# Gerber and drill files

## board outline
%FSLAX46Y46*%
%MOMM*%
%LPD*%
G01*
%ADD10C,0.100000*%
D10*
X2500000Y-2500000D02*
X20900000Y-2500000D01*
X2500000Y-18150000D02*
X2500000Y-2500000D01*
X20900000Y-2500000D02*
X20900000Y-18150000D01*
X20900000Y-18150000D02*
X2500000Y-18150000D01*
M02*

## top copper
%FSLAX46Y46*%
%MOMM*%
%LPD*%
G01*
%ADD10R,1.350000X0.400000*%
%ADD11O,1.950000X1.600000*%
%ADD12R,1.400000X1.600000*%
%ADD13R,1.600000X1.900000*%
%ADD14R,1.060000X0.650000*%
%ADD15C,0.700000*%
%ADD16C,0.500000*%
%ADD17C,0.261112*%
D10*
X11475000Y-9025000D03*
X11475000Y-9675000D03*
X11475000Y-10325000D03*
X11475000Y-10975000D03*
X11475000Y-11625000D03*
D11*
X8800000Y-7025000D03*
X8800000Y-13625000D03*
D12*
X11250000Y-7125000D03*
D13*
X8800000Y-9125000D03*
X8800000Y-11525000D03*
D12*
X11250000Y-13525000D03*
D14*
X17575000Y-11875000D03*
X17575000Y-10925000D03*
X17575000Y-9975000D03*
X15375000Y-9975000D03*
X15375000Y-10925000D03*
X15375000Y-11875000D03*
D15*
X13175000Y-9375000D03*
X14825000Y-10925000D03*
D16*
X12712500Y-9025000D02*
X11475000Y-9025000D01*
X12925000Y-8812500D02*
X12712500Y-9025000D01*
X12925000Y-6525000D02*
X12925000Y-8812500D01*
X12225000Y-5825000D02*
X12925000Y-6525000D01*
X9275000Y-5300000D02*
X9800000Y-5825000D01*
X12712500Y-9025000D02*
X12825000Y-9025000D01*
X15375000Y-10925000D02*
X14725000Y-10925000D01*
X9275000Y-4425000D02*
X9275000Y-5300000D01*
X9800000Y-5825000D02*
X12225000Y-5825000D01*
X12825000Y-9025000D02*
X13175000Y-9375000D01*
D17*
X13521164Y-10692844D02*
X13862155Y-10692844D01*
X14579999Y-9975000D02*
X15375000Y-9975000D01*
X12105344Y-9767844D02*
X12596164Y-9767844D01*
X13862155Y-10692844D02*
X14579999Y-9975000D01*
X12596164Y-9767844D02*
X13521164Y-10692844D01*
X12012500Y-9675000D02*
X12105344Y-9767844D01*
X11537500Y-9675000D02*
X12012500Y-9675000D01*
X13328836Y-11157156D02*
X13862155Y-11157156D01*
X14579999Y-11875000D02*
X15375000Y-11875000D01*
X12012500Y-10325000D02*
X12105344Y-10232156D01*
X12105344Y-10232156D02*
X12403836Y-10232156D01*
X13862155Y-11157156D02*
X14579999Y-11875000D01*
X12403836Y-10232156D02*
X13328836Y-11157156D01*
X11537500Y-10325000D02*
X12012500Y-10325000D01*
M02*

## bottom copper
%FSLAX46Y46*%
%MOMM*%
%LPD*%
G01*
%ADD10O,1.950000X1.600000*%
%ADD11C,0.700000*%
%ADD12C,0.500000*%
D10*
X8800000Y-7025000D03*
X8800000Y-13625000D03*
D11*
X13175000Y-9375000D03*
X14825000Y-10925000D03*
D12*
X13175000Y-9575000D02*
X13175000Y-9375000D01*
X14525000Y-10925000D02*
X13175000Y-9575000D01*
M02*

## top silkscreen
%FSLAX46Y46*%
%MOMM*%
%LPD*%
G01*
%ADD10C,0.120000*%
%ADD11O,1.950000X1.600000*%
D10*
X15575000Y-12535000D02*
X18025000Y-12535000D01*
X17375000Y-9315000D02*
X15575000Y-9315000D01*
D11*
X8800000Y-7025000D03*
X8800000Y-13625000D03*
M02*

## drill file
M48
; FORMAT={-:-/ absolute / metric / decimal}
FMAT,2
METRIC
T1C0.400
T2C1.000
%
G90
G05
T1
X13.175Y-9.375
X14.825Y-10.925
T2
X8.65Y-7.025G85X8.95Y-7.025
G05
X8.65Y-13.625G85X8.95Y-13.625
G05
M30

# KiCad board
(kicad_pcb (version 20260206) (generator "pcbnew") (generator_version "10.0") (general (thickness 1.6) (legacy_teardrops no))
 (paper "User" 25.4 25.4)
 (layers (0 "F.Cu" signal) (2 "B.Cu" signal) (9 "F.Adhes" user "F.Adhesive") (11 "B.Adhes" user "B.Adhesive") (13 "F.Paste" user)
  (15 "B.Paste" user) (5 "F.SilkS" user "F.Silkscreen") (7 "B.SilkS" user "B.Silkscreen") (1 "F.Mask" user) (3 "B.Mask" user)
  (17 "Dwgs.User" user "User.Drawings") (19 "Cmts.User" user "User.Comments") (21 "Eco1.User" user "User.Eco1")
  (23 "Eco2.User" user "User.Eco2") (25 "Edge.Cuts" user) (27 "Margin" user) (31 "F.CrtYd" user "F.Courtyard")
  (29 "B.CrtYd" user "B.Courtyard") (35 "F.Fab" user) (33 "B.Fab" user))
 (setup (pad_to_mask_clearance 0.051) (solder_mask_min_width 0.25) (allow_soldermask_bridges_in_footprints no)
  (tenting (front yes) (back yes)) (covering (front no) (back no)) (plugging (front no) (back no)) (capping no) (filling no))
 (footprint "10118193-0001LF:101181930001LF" (layer "F.Cu") (at 8.875 10.325 -90)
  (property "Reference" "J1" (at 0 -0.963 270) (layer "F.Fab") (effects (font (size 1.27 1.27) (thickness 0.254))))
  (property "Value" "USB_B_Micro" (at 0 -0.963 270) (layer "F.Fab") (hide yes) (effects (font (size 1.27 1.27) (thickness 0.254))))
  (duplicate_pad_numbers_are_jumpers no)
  (pad "1" smd rect (at -1.3 -2.6 270) (size 0.4 1.35) (layers "F.Cu" "F.Mask" "F.Paste") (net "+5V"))
  (pad "2" smd rect (at -0.65 -2.6 270) (size 0.4 1.35) (layers "F.Cu" "F.Mask" "F.Paste") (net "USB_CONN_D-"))
  (pad "3" smd rect (at 0 -2.6 270) (size 0.4 1.35) (layers "F.Cu" "F.Mask" "F.Paste") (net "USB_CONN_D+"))
  (pad "4" smd rect (at 0.65 -2.6 270) (size 0.4 1.35) (layers "F.Cu" "F.Mask" "F.Paste") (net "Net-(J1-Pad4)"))
  (pad "5" smd rect (at 1.3 -2.6 270) (size 0.4 1.35) (layers "F.Cu" "F.Mask" "F.Paste") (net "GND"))
  (pad "MH1" thru_hole oval (at -3.3 0.075) (size 1.95 1.6) (drill oval 1.3 1) (layers "*.Cu" "*.Mask" "F.SilkS") (remove_unused_layers no))
  (pad "MH2" thru_hole oval (at 3.3 0.075) (size 1.95 1.6) (drill oval 1.3 1) (layers "*.Cu" "*.Mask" "F.SilkS") (remove_unused_layers no))
  (pad "MP1" smd rect (at -3.2 -2.375) (size 1.4 1.6) (layers "F.Cu" "F.Mask" "F.Paste"))
  (pad "MP2" smd rect (at -1.2 0.075) (size 1.6 1.9) (layers "F.Cu" "F.Mask" "F.Paste"))
  (pad "MP3" smd rect (at 1.2 0.075) (size 1.6 1.9) (layers "F.Cu" "F.Mask" "F.Paste"))
  (pad "MP4" smd rect (at 3.2 -2.375) (size 1.4 1.6) (layers "F.Cu" "F.Mask" "F.Paste")))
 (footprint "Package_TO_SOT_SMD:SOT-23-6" (layer "F.Cu") (at 16.475 10.925 180)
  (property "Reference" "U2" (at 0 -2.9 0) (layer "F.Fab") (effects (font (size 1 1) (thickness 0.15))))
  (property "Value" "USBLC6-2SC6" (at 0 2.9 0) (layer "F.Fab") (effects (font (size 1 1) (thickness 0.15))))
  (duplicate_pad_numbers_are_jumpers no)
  (fp_line (start 0.9 -1.61) (end -1.55 -1.61) (stroke (width 0.12) (type solid)) (layer "F.SilkS"))
  (fp_line (start -0.9 1.61) (end 0.9 1.61) (stroke (width 0.12) (type solid)) (layer "F.SilkS"))
  (pad "1" smd rect (at -1.1 -0.95 180) (size 1.06 0.65) (layers "F.Cu" "F.Mask" "F.Paste") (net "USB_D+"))
  (pad "2" smd rect (at -1.1 0 180) (size 1.06 0.65) (layers "F.Cu" "F.Mask" "F.Paste") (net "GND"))
  (pad "3" smd rect (at -1.1 0.95 180) (size 1.06 0.65) (layers "F.Cu" "F.Mask" "F.Paste") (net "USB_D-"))
  (pad "4" smd rect (at 1.1 0.95 180) (size 1.06 0.65) (layers "F.Cu" "F.Mask" "F.Paste") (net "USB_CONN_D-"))
  (pad "5" smd rect (at 1.1 0 180) (size 1.06 0.65) (layers "F.Cu" "F.Mask" "F.Paste") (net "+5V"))
  (pad "6" smd rect (at 1.1 -0.95 180) (size 1.06 0.65) (layers "F.Cu" "F.Mask" "F.Paste") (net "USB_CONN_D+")))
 (gr_line (start 2.5 2.5) (end 20.9 2.5) (stroke (width 0.1) (type default)) (layer "Edge.Cuts"))
 (gr_line (start 2.5 18.15) (end 2.5 2.5) (stroke (width 0.1) (type default)) (layer "Edge.Cuts"))
 (gr_line (start 20.9 2.5) (end 20.9 18.15) (stroke (width 0.1) (type default)) (layer "Edge.Cuts"))
 (gr_line (start 20.9 18.15) (end 2.5 18.15) (stroke (width 0.1) (type default)) (layer "Edge.Cuts"))
 (segment (start 12.7125 9.025) (end 11.475 9.025) (width 0.5) (layer "F.Cu") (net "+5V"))
 (segment (start 12.925 8.8125) (end 12.7125 9.025) (width 0.5) (layer "F.Cu") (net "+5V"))
 (segment (start 12.925 6.525) (end 12.925 8.8125) (width 0.5) (layer "F.Cu") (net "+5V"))
 (segment (start 12.225 5.825) (end 12.925 6.525) (width 0.5) (layer "F.Cu") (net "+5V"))
 (segment (start 9.275 5.3) (end 9.8 5.825) (width 0.5) (layer "F.Cu") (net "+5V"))
 (segment (start 12.7125 9.025) (end 12.825 9.025) (width 0.5) (layer "F.Cu") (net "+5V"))
 (segment (start 15.375 10.925) (end 14.725 10.925) (width 0.5) (layer "F.Cu") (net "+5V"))
 (segment (start 9.275 4.425) (end 9.275 5.3) (width 0.5) (layer "F.Cu") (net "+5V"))
 (segment (start 9.8 5.825) (end 12.225 5.825) (width 0.5) (layer "F.Cu") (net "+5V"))
 (segment (start 12.825 9.025) (end 13.175 9.375) (width 0.5) (layer "F.Cu") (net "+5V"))
 (via (at 13.175 9.375) (size 0.7) (drill 0.4) (layers "F.Cu" "B.Cu") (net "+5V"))
 (via (at 14.825 10.925) (size 0.7) (drill 0.4) (layers "F.Cu" "B.Cu") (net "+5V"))
 (segment (start 13.175 9.575) (end 13.175 9.375) (width 0.5) (layer "B.Cu") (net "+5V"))
 (segment (start 14.525 10.925) (end 13.175 9.575) (width 0.5) (layer "B.Cu") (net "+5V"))
 (segment (start 13.521164 10.692844) (end 13.862155 10.692844) (width 0.261112) (layer "F.Cu") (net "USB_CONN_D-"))
 (segment (start 14.579999 9.975) (end 15.375 9.975) (width 0.261112) (layer "F.Cu") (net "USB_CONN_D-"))
 (segment (start 12.105344 9.767844) (end 12.596164 9.767844) (width 0.261112) (layer "F.Cu") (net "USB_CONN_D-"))
 (segment (start 13.862155 10.692844) (end 14.579999 9.975) (width 0.261112) (layer "F.Cu") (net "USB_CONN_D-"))
 (segment (start 12.596164 9.767844) (end 13.521164 10.692844) (width 0.261112) (layer "F.Cu") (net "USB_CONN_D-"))
 (segment (start 12.0125 9.675) (end 12.105344 9.767844) (width 0.261112) (layer "F.Cu") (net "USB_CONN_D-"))
 (segment (start 11.5375 9.675) (end 12.0125 9.675) (width 0.261112) (layer "F.Cu") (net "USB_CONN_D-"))
 (segment (start 13.328836 11.157156) (end 13.862155 11.157156) (width 0.261112) (layer "F.Cu") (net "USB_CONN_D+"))
 (segment (start 14.579999 11.875) (end 15.375 11.875) (width 0.261112) (layer "F.Cu") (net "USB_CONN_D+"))
 (segment (start 12.0125 10.325) (end 12.105344 10.232156) (width 0.261112) (layer "F.Cu") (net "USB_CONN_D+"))
 (segment (start 12.105344 10.232156) (end 12.403836 10.232156) (width 0.261112) (layer "F.Cu") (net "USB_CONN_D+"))
 (segment (start 13.862155 11.157156) (end 14.579999 11.875) (width 0.261112) (layer "F.Cu") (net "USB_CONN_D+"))
 (segment (start 12.403836 10.232156) (end 13.328836 11.157156) (width 0.261112) (layer "F.Cu") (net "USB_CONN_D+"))
 (segment (start 11.5375 10.325) (end 12.0125 10.325) (width 0.261112) (layer "F.Cu") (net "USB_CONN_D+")))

